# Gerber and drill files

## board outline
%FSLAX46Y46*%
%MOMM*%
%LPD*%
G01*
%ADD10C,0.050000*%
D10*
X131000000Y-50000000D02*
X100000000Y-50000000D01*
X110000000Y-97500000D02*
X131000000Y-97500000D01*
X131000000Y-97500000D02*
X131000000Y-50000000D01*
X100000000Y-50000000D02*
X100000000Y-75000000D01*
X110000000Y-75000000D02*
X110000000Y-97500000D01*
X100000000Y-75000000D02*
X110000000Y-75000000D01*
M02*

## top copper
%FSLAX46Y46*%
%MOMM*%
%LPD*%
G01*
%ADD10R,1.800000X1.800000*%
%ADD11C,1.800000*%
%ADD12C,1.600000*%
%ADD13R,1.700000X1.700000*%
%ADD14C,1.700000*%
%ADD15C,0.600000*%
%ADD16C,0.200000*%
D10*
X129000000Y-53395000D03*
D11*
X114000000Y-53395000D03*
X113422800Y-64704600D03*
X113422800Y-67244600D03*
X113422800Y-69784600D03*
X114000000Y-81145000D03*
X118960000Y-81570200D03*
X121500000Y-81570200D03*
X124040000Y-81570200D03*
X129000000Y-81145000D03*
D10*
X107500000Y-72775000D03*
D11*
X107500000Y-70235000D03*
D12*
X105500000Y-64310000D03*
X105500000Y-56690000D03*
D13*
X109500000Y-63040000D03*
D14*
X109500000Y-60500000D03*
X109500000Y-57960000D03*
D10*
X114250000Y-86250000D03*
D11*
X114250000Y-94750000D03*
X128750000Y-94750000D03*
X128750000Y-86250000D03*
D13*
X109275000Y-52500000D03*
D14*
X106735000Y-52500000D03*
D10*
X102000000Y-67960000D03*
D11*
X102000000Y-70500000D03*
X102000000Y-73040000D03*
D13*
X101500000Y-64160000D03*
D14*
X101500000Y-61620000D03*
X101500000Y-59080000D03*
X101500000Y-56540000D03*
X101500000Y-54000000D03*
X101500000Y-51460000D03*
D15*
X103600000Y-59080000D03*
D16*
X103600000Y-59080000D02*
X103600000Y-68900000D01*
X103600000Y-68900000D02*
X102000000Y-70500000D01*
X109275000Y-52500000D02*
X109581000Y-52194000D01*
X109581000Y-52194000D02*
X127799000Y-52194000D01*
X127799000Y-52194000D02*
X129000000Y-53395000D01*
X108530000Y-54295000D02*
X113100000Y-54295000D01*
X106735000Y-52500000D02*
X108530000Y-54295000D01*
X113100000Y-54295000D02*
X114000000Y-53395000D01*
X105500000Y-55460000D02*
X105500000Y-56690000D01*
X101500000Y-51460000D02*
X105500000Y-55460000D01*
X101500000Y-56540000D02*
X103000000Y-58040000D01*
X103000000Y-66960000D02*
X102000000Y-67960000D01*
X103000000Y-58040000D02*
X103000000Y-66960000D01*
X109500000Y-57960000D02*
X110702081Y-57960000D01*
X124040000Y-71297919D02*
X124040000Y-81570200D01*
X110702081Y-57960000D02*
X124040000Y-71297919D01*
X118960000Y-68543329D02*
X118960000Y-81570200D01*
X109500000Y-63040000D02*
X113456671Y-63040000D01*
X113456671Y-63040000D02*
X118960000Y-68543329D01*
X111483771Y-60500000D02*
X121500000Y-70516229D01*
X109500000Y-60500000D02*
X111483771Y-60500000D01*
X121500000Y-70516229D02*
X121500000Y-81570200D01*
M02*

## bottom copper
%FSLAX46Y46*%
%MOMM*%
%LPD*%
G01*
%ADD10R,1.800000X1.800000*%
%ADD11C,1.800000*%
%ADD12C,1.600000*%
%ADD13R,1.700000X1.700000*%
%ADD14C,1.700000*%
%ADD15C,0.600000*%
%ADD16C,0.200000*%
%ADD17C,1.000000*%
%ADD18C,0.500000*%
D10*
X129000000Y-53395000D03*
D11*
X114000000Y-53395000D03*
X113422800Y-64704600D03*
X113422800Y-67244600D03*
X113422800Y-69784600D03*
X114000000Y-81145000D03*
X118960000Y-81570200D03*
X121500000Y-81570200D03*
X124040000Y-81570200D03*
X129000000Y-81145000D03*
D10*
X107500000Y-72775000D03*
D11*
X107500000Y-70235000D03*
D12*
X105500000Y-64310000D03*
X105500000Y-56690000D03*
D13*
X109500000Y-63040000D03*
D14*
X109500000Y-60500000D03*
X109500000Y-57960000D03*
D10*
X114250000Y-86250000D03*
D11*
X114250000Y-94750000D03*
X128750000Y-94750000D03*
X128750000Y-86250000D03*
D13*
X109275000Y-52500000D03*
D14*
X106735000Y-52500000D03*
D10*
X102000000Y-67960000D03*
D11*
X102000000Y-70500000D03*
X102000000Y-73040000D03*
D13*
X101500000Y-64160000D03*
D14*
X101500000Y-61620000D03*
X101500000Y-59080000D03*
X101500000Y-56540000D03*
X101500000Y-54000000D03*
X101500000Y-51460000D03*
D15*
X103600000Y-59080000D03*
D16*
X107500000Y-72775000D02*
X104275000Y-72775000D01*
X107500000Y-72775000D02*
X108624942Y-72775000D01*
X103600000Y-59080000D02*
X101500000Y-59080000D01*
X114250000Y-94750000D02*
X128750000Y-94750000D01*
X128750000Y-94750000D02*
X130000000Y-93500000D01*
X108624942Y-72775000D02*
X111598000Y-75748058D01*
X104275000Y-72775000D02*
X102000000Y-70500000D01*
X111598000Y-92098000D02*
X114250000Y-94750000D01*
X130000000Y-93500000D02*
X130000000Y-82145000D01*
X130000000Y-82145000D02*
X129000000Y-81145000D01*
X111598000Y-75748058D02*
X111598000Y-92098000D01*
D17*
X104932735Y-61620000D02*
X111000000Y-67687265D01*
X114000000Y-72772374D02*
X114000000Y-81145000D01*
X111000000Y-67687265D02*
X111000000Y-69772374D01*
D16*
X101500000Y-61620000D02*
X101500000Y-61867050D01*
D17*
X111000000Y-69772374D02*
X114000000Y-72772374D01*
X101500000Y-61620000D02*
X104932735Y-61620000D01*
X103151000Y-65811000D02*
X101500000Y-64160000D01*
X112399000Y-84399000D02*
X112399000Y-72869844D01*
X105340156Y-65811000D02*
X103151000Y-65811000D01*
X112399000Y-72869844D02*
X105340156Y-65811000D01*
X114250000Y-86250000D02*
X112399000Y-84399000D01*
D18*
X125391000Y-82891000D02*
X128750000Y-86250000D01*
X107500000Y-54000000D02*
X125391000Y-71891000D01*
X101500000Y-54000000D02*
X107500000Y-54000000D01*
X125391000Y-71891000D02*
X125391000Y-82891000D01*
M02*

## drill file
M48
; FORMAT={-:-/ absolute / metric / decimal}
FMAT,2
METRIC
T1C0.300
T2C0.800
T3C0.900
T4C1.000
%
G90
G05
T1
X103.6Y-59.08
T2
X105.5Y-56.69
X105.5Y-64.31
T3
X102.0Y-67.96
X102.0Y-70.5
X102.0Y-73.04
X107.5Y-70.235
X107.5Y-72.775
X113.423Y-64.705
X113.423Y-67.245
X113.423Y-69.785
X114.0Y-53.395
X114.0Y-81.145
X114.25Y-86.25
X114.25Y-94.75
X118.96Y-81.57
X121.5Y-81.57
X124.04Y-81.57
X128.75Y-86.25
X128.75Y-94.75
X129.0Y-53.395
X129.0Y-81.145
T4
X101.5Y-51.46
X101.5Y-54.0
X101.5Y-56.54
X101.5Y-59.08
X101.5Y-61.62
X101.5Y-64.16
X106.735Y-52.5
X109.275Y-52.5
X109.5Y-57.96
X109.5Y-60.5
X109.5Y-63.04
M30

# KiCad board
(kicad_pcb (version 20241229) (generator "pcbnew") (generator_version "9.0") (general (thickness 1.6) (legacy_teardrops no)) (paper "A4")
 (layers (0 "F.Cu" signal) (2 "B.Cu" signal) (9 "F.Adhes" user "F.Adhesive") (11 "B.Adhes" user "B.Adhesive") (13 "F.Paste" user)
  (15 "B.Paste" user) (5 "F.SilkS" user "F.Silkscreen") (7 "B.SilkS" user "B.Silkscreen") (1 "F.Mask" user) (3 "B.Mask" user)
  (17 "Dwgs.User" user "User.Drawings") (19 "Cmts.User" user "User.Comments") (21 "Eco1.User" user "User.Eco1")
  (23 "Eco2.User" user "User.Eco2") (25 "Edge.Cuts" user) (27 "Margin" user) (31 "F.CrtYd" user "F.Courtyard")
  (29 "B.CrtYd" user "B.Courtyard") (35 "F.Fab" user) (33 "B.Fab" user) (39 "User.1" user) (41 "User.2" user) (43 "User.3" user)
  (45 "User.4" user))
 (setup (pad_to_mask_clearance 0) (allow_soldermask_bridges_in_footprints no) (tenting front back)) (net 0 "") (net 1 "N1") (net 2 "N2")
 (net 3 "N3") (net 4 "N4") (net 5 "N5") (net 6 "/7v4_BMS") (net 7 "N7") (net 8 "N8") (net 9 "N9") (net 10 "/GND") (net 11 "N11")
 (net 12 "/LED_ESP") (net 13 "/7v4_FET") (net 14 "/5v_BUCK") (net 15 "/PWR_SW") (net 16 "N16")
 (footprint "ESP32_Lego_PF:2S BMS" (layer "F.Cu") (at 121.5 67.27)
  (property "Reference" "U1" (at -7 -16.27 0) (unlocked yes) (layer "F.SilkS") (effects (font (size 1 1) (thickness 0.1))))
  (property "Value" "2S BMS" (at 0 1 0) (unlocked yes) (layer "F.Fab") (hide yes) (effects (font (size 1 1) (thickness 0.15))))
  (pad "1" thru_hole rect (at 7.5 -13.875) (size 1.8 1.8) (drill 0.9) (layers "*.Cu" "*.Mask") (remove_unused_layers no) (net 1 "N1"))
  (pad "2" thru_hole circle (at -7.5 -13.875) (size 1.8 1.8) (drill 0.9) (layers "*.Cu" "*.Mask") (remove_unused_layers no) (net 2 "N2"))
  (pad "3" thru_hole circle (at -8.0772 -2.5654) (size 1.8 1.8) (drill 0.9) (layers "*.Cu" "*.Mask") (remove_unused_layers no) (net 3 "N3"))
  (pad "4" thru_hole circle (at -8.0772 -0.0254) (size 1.8 1.8) (drill 0.9) (layers "*.Cu" "*.Mask") (remove_unused_layers no) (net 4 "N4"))
  (pad "5" thru_hole circle (at -8.0772 2.5146) (size 1.8 1.8) (drill 0.9) (layers "*.Cu" "*.Mask") (remove_unused_layers no) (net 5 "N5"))
  (pad "6" thru_hole circle (at -7.5 13.875) (size 1.8 1.8) (drill 0.9) (layers "*.Cu" "*.Mask") (remove_unused_layers no)
   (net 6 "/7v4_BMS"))
  (pad "7" thru_hole circle (at -2.54 14.3002) (size 1.8 1.8) (drill 0.9) (layers "*.Cu" "*.Mask") (remove_unused_layers no) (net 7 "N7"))
  (pad "8" thru_hole circle (at 0 14.3002) (size 1.8 1.8) (drill 0.9) (layers "*.Cu" "*.Mask") (remove_unused_layers no) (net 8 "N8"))
  (pad "9" thru_hole circle (at 2.54 14.3002) (size 1.8 1.8) (drill 0.9) (layers "*.Cu" "*.Mask") (remove_unused_layers no) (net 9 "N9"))
  (pad "10" thru_hole circle (at 7.5 13.875) (size 1.8 1.8) (drill 0.9) (layers "*.Cu" "*.Mask") (remove_unused_layers no) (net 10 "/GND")))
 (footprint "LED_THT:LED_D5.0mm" (layer "F.Cu") (at 107.5 72.775 90)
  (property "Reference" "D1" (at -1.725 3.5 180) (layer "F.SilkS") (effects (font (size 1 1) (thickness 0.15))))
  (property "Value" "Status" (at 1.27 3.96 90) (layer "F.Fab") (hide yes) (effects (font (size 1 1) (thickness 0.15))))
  (pad "1" thru_hole rect (at 0 0 90) (size 1.8 1.8) (drill 0.9) (layers "*.Cu" "*.Mask") (remove_unused_layers no) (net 10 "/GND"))
  (pad "2" thru_hole circle (at 2.54 0 90) (size 1.8 1.8) (drill 0.9) (layers "*.Cu" "*.Mask") (remove_unused_layers no) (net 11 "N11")))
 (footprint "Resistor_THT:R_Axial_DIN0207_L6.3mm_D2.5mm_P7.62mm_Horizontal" (layer "F.Cu") (at 105.5 64.31 90)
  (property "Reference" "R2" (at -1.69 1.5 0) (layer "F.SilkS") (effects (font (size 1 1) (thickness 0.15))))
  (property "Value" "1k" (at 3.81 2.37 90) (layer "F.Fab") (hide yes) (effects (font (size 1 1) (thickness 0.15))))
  (pad "1" thru_hole circle (at 0 0 90) (size 1.6 1.6) (drill 0.8) (layers "*.Cu" "*.Mask") (remove_unused_layers no) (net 11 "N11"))
  (pad "2" thru_hole circle (at 7.62 0 90) (size 1.6 1.6) (drill 0.8) (layers "*.Cu" "*.Mask") (remove_unused_layers no) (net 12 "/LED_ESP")))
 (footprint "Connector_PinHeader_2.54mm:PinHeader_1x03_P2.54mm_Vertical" (layer "F.Cu") (at 109.5 63.04 180)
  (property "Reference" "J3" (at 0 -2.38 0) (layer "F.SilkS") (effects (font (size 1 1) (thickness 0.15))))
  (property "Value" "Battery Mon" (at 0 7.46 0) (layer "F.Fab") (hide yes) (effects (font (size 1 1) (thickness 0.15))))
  (pad "1" thru_hole rect (at 0 0 180) (size 1.7 1.7) (drill 1) (layers "*.Cu" "*.Mask") (remove_unused_layers no) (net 7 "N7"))
  (pad "2" thru_hole circle (at 0 2.54 180) (size 1.7 1.7) (drill 1) (layers "*.Cu" "*.Mask") (remove_unused_layers no) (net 8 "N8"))
  (pad "3" thru_hole circle (at 0 5.08 180) (size 1.7 1.7) (drill 1) (layers "*.Cu" "*.Mask") (remove_unused_layers no) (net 9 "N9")))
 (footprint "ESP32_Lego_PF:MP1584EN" (layer "F.Cu") (at 121.5 90.5 90)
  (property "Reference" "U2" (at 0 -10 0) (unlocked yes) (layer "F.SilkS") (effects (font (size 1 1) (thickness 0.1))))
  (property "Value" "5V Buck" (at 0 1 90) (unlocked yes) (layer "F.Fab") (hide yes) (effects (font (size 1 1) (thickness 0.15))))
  (pad "1" thru_hole rect (at 4.25 -7.25 90) (size 1.8 1.8) (drill 0.9) (layers "*.Cu" "*.Mask") (remove_unused_layers no)
   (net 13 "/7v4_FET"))
  (pad "2" thru_hole circle (at -4.25 -7.25 90) (size 1.8 1.8) (drill 0.9) (layers "*.Cu" "*.Mask") (remove_unused_layers no)
   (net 10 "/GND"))
  (pad "3" thru_hole circle (at -4.25 7.25 90) (size 1.8 1.8) (drill 0.9) (layers "*.Cu" "*.Mask") (remove_unused_layers no) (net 10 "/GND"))
  (pad "4" thru_hole circle (at 4.25 7.25 90) (size 1.8 1.8) (drill 0.9) (layers "*.Cu" "*.Mask") (remove_unused_layers no)
   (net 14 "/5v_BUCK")))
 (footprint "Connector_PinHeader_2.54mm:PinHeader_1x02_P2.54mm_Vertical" (layer "F.Cu") (at 109.275 52.5 -90)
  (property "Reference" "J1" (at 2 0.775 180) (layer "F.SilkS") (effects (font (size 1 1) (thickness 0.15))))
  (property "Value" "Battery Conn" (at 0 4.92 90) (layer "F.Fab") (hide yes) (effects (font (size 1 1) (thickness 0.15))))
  (pad "1" thru_hole rect (at 0 0 270) (size 1.7 1.7) (drill 1) (layers "*.Cu" "*.Mask") (remove_unused_layers no) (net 1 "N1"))
  (pad "2" thru_hole circle (at 0 2.54 270) (size 1.7 1.7) (drill 1) (layers "*.Cu" "*.Mask") (remove_unused_layers no) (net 2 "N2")))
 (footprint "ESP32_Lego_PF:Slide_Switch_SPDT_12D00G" (layer "F.Cu") (at 102 70.5)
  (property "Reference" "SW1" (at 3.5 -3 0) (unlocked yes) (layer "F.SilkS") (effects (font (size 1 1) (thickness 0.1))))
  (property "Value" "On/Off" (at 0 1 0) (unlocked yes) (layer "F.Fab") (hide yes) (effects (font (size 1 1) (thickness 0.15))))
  (pad "1" thru_hole rect (at 0 -2.54) (size 1.8 1.8) (drill 0.9) (layers "*.Cu" "*.Mask") (remove_unused_layers no) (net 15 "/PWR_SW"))
  (pad "2" thru_hole circle (at 0 0) (size 1.8 1.8) (drill 0.9) (layers "*.Cu" "*.Mask") (remove_unused_layers no) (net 10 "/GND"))
  (pad "3" thru_hole circle (at 0 2.54) (size 1.8 1.8) (drill 0.9) (layers "*.Cu" "*.Mask") (remove_unused_layers no) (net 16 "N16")))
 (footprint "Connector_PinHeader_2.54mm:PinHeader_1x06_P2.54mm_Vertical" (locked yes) (layer "B.Cu") (at 101.5 64.16)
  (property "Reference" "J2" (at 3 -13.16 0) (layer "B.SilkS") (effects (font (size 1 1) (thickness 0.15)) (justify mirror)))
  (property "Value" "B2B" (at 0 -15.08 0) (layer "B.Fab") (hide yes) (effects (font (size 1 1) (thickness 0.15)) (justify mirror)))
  (pad "1" thru_hole rect (at 0 0) (size 1.7 1.7) (drill 1) (layers "*.Cu" "*.Mask") (remove_unused_layers no) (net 13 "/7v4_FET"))
  (pad "2" thru_hole circle (at 0 -2.54) (size 1.7 1.7) (drill 1) (layers "*.Cu" "*.Mask") (remove_unused_layers no) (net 6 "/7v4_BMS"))
  (pad "3" thru_hole circle (at 0 -5.08) (size 1.7 1.7) (drill 1) (layers "*.Cu" "*.Mask") (remove_unused_layers no) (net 10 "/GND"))
  (pad "4" thru_hole circle (at 0 -7.62) (size 1.7 1.7) (drill 1) (layers "*.Cu" "*.Mask") (remove_unused_layers no) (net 15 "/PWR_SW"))
  (pad "5" thru_hole circle (at 0 -10.16) (size 1.7 1.7) (drill 1) (layers "*.Cu" "*.Mask") (remove_unused_layers no) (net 14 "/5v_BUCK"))
  (pad "6" thru_hole circle (at 0 -12.7) (size 1.7 1.7) (drill 1) (layers "*.Cu" "*.Mask") (remove_unused_layers no) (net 12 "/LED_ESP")))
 (gr_line (start 131 50) (end 100 50) (stroke (width 0.05) (type default)) (layer "Edge.Cuts"))
 (gr_line (start 110 97.5) (end 131 97.5) (stroke (width 0.05) (type default)) (layer "Edge.Cuts"))
 (gr_line (start 131 97.5) (end 131 50) (stroke (width 0.05) (type default)) (layer "Edge.Cuts"))
 (gr_line (start 100 50) (end 100 75) (stroke (width 0.05) (type default)) (layer "Edge.Cuts"))
 (gr_line (start 110 75) (end 110 97.5) (stroke (width 0.05) (type default)) (layer "Edge.Cuts"))
 (gr_line (start 100 75) (end 110 75) (stroke (width 0.05) (type default)) (layer "Edge.Cuts"))
 (segment (start 103.6 59.08) (end 103.6 68.9) (width 0.2) (layer "F.Cu") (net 10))
 (segment (start 103.6 68.9) (end 102 70.5) (width 0.2) (layer "F.Cu") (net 10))
 (via (at 103.6 59.08) (size 0.6) (drill 0.3) (layers "F.Cu" "B.Cu") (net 10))
 (segment (start 107.5 72.775) (end 104.275 72.775) (width 0.2) (layer "B.Cu") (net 10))
 (segment (start 107.5 72.775) (end 108.624942 72.775) (width 0.2) (layer "B.Cu") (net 10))
 (segment (start 103.6 59.08) (end 101.5 59.08) (width 0.2) (layer "B.Cu") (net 10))
 (segment (start 114.25 94.75) (end 128.75 94.75) (width 0.2) (layer "B.Cu") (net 10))
 (segment (start 128.75 94.75) (end 130 93.5) (width 0.2) (layer "B.Cu") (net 10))
 (segment (start 108.624942 72.775) (end 111.598 75.748058) (width 0.2) (layer "B.Cu") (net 10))
 (segment (start 104.275 72.775) (end 102 70.5) (width 0.2) (layer "B.Cu") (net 10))
 (segment (start 111.598 92.098) (end 114.25 94.75) (width 0.2) (layer "B.Cu") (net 10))
 (segment (start 130 93.5) (end 130 82.145) (width 0.2) (layer "B.Cu") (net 10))
 (segment (start 130 82.145) (end 129 81.145) (width 0.2) (layer "B.Cu") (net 10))
 (segment (start 111.598 75.748058) (end 111.598 92.098) (width 0.2) (layer "B.Cu") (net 10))
 (segment (start 109.275 52.5) (end 109.581 52.194) (width 0.2) (layer "F.Cu") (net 1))
 (segment (start 109.581 52.194) (end 127.799 52.194) (width 0.2) (layer "F.Cu") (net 1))
 (segment (start 127.799 52.194) (end 129 53.395) (width 0.2) (layer "F.Cu") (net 1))
 (segment (start 108.53 54.295) (end 113.1 54.295) (width 0.2) (layer "F.Cu") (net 2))
 (segment (start 106.735 52.5) (end 108.53 54.295) (width 0.2) (layer "F.Cu") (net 2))
 (segment (start 113.1 54.295) (end 114 53.395) (width 0.2) (layer "F.Cu") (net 2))
 (segment (start 105.5 55.46) (end 105.5 56.69) (width 0.2) (layer "F.Cu") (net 12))
 (segment (start 101.5 51.46) (end 105.5 55.46) (width 0.2) (layer "F.Cu") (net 12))
 (segment (start 101.5 56.54) (end 103 58.04) (width 0.2) (layer "F.Cu") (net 15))
 (segment (start 103 66.96) (end 102 67.96) (width 0.2) (layer "F.Cu") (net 15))
 (segment (start 103 58.04) (end 103 66.96) (width 0.2) (layer "F.Cu") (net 15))
 (segment (start 109.5 57.96) (end 110.702081 57.96) (width 0.2) (layer "F.Cu") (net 9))
 (segment (start 124.04 71.297919) (end 124.04 81.5702) (width 0.2) (layer "F.Cu") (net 9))
 (segment (start 110.702081 57.96) (end 124.04 71.297919) (width 0.2) (layer "F.Cu") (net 9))
 (segment (start 104.932735 61.62) (end 111 67.687265) (width 1) (layer "B.Cu") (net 6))
 (segment (start 114 72.772374) (end 114 81.145) (width 1) (layer "B.Cu") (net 6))
 (segment (start 111 67.687265) (end 111 69.772374) (width 1) (layer "B.Cu") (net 6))
 (segment (start 101.5 61.62) (end 101.5 61.86705) (width 0.2) (layer "B.Cu") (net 6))
 (segment (start 111 69.772374) (end 114 72.772374) (width 1) (layer "B.Cu") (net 6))
 (segment (start 101.5 61.62) (end 104.932735 61.62) (width 1) (layer "B.Cu") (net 6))
 (segment (start 118.96 68.543329) (end 118.96 81.5702) (width 0.2) (layer "F.Cu") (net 7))
 (segment (start 109.5 63.04) (end 113.456671 63.04) (width 0.2) (layer "F.Cu") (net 7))
 (segment (start 113.456671 63.04) (end 118.96 68.543329) (width 0.2) (layer "F.Cu") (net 7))
 (segment (start 111.483771 60.5) (end 121.5 70.516229) (width 0.2) (layer "F.Cu") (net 8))
 (segment (start 109.5 60.5) (end 111.483771 60.5) (width 0.2) (layer "F.Cu") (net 8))
 (segment (start 121.5 70.516229) (end 121.5 81.5702) (width 0.2) (layer "F.Cu") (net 8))
 (segment (start 103.151 65.811) (end 101.5 64.16) (width 1) (layer "B.Cu") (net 13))
 (segment (start 112.399 84.399) (end 112.399 72.869844) (width 1) (layer "B.Cu") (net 13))
 (segment (start 105.340156 65.811) (end 103.151 65.811) (width 1) (layer "B.Cu") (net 13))
 (segment (start 112.399 72.869844) (end 105.340156 65.811) (width 1) (layer "B.Cu") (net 13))
 (segment (start 114.25 86.25) (end 112.399 84.399) (width 1) (layer "B.Cu") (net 13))
 (segment (start 125.391 82.891) (end 128.75 86.25) (width 0.5) (layer "B.Cu") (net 14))
 (segment (start 107.5 54) (end 125.391 71.891) (width 0.5) (layer "B.Cu") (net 14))
 (segment (start 101.5 54) (end 107.5 54) (width 0.5) (layer "B.Cu") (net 14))
 (segment (start 125.391 71.891) (end 125.391 82.891) (width 0.5) (layer "B.Cu") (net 14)))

